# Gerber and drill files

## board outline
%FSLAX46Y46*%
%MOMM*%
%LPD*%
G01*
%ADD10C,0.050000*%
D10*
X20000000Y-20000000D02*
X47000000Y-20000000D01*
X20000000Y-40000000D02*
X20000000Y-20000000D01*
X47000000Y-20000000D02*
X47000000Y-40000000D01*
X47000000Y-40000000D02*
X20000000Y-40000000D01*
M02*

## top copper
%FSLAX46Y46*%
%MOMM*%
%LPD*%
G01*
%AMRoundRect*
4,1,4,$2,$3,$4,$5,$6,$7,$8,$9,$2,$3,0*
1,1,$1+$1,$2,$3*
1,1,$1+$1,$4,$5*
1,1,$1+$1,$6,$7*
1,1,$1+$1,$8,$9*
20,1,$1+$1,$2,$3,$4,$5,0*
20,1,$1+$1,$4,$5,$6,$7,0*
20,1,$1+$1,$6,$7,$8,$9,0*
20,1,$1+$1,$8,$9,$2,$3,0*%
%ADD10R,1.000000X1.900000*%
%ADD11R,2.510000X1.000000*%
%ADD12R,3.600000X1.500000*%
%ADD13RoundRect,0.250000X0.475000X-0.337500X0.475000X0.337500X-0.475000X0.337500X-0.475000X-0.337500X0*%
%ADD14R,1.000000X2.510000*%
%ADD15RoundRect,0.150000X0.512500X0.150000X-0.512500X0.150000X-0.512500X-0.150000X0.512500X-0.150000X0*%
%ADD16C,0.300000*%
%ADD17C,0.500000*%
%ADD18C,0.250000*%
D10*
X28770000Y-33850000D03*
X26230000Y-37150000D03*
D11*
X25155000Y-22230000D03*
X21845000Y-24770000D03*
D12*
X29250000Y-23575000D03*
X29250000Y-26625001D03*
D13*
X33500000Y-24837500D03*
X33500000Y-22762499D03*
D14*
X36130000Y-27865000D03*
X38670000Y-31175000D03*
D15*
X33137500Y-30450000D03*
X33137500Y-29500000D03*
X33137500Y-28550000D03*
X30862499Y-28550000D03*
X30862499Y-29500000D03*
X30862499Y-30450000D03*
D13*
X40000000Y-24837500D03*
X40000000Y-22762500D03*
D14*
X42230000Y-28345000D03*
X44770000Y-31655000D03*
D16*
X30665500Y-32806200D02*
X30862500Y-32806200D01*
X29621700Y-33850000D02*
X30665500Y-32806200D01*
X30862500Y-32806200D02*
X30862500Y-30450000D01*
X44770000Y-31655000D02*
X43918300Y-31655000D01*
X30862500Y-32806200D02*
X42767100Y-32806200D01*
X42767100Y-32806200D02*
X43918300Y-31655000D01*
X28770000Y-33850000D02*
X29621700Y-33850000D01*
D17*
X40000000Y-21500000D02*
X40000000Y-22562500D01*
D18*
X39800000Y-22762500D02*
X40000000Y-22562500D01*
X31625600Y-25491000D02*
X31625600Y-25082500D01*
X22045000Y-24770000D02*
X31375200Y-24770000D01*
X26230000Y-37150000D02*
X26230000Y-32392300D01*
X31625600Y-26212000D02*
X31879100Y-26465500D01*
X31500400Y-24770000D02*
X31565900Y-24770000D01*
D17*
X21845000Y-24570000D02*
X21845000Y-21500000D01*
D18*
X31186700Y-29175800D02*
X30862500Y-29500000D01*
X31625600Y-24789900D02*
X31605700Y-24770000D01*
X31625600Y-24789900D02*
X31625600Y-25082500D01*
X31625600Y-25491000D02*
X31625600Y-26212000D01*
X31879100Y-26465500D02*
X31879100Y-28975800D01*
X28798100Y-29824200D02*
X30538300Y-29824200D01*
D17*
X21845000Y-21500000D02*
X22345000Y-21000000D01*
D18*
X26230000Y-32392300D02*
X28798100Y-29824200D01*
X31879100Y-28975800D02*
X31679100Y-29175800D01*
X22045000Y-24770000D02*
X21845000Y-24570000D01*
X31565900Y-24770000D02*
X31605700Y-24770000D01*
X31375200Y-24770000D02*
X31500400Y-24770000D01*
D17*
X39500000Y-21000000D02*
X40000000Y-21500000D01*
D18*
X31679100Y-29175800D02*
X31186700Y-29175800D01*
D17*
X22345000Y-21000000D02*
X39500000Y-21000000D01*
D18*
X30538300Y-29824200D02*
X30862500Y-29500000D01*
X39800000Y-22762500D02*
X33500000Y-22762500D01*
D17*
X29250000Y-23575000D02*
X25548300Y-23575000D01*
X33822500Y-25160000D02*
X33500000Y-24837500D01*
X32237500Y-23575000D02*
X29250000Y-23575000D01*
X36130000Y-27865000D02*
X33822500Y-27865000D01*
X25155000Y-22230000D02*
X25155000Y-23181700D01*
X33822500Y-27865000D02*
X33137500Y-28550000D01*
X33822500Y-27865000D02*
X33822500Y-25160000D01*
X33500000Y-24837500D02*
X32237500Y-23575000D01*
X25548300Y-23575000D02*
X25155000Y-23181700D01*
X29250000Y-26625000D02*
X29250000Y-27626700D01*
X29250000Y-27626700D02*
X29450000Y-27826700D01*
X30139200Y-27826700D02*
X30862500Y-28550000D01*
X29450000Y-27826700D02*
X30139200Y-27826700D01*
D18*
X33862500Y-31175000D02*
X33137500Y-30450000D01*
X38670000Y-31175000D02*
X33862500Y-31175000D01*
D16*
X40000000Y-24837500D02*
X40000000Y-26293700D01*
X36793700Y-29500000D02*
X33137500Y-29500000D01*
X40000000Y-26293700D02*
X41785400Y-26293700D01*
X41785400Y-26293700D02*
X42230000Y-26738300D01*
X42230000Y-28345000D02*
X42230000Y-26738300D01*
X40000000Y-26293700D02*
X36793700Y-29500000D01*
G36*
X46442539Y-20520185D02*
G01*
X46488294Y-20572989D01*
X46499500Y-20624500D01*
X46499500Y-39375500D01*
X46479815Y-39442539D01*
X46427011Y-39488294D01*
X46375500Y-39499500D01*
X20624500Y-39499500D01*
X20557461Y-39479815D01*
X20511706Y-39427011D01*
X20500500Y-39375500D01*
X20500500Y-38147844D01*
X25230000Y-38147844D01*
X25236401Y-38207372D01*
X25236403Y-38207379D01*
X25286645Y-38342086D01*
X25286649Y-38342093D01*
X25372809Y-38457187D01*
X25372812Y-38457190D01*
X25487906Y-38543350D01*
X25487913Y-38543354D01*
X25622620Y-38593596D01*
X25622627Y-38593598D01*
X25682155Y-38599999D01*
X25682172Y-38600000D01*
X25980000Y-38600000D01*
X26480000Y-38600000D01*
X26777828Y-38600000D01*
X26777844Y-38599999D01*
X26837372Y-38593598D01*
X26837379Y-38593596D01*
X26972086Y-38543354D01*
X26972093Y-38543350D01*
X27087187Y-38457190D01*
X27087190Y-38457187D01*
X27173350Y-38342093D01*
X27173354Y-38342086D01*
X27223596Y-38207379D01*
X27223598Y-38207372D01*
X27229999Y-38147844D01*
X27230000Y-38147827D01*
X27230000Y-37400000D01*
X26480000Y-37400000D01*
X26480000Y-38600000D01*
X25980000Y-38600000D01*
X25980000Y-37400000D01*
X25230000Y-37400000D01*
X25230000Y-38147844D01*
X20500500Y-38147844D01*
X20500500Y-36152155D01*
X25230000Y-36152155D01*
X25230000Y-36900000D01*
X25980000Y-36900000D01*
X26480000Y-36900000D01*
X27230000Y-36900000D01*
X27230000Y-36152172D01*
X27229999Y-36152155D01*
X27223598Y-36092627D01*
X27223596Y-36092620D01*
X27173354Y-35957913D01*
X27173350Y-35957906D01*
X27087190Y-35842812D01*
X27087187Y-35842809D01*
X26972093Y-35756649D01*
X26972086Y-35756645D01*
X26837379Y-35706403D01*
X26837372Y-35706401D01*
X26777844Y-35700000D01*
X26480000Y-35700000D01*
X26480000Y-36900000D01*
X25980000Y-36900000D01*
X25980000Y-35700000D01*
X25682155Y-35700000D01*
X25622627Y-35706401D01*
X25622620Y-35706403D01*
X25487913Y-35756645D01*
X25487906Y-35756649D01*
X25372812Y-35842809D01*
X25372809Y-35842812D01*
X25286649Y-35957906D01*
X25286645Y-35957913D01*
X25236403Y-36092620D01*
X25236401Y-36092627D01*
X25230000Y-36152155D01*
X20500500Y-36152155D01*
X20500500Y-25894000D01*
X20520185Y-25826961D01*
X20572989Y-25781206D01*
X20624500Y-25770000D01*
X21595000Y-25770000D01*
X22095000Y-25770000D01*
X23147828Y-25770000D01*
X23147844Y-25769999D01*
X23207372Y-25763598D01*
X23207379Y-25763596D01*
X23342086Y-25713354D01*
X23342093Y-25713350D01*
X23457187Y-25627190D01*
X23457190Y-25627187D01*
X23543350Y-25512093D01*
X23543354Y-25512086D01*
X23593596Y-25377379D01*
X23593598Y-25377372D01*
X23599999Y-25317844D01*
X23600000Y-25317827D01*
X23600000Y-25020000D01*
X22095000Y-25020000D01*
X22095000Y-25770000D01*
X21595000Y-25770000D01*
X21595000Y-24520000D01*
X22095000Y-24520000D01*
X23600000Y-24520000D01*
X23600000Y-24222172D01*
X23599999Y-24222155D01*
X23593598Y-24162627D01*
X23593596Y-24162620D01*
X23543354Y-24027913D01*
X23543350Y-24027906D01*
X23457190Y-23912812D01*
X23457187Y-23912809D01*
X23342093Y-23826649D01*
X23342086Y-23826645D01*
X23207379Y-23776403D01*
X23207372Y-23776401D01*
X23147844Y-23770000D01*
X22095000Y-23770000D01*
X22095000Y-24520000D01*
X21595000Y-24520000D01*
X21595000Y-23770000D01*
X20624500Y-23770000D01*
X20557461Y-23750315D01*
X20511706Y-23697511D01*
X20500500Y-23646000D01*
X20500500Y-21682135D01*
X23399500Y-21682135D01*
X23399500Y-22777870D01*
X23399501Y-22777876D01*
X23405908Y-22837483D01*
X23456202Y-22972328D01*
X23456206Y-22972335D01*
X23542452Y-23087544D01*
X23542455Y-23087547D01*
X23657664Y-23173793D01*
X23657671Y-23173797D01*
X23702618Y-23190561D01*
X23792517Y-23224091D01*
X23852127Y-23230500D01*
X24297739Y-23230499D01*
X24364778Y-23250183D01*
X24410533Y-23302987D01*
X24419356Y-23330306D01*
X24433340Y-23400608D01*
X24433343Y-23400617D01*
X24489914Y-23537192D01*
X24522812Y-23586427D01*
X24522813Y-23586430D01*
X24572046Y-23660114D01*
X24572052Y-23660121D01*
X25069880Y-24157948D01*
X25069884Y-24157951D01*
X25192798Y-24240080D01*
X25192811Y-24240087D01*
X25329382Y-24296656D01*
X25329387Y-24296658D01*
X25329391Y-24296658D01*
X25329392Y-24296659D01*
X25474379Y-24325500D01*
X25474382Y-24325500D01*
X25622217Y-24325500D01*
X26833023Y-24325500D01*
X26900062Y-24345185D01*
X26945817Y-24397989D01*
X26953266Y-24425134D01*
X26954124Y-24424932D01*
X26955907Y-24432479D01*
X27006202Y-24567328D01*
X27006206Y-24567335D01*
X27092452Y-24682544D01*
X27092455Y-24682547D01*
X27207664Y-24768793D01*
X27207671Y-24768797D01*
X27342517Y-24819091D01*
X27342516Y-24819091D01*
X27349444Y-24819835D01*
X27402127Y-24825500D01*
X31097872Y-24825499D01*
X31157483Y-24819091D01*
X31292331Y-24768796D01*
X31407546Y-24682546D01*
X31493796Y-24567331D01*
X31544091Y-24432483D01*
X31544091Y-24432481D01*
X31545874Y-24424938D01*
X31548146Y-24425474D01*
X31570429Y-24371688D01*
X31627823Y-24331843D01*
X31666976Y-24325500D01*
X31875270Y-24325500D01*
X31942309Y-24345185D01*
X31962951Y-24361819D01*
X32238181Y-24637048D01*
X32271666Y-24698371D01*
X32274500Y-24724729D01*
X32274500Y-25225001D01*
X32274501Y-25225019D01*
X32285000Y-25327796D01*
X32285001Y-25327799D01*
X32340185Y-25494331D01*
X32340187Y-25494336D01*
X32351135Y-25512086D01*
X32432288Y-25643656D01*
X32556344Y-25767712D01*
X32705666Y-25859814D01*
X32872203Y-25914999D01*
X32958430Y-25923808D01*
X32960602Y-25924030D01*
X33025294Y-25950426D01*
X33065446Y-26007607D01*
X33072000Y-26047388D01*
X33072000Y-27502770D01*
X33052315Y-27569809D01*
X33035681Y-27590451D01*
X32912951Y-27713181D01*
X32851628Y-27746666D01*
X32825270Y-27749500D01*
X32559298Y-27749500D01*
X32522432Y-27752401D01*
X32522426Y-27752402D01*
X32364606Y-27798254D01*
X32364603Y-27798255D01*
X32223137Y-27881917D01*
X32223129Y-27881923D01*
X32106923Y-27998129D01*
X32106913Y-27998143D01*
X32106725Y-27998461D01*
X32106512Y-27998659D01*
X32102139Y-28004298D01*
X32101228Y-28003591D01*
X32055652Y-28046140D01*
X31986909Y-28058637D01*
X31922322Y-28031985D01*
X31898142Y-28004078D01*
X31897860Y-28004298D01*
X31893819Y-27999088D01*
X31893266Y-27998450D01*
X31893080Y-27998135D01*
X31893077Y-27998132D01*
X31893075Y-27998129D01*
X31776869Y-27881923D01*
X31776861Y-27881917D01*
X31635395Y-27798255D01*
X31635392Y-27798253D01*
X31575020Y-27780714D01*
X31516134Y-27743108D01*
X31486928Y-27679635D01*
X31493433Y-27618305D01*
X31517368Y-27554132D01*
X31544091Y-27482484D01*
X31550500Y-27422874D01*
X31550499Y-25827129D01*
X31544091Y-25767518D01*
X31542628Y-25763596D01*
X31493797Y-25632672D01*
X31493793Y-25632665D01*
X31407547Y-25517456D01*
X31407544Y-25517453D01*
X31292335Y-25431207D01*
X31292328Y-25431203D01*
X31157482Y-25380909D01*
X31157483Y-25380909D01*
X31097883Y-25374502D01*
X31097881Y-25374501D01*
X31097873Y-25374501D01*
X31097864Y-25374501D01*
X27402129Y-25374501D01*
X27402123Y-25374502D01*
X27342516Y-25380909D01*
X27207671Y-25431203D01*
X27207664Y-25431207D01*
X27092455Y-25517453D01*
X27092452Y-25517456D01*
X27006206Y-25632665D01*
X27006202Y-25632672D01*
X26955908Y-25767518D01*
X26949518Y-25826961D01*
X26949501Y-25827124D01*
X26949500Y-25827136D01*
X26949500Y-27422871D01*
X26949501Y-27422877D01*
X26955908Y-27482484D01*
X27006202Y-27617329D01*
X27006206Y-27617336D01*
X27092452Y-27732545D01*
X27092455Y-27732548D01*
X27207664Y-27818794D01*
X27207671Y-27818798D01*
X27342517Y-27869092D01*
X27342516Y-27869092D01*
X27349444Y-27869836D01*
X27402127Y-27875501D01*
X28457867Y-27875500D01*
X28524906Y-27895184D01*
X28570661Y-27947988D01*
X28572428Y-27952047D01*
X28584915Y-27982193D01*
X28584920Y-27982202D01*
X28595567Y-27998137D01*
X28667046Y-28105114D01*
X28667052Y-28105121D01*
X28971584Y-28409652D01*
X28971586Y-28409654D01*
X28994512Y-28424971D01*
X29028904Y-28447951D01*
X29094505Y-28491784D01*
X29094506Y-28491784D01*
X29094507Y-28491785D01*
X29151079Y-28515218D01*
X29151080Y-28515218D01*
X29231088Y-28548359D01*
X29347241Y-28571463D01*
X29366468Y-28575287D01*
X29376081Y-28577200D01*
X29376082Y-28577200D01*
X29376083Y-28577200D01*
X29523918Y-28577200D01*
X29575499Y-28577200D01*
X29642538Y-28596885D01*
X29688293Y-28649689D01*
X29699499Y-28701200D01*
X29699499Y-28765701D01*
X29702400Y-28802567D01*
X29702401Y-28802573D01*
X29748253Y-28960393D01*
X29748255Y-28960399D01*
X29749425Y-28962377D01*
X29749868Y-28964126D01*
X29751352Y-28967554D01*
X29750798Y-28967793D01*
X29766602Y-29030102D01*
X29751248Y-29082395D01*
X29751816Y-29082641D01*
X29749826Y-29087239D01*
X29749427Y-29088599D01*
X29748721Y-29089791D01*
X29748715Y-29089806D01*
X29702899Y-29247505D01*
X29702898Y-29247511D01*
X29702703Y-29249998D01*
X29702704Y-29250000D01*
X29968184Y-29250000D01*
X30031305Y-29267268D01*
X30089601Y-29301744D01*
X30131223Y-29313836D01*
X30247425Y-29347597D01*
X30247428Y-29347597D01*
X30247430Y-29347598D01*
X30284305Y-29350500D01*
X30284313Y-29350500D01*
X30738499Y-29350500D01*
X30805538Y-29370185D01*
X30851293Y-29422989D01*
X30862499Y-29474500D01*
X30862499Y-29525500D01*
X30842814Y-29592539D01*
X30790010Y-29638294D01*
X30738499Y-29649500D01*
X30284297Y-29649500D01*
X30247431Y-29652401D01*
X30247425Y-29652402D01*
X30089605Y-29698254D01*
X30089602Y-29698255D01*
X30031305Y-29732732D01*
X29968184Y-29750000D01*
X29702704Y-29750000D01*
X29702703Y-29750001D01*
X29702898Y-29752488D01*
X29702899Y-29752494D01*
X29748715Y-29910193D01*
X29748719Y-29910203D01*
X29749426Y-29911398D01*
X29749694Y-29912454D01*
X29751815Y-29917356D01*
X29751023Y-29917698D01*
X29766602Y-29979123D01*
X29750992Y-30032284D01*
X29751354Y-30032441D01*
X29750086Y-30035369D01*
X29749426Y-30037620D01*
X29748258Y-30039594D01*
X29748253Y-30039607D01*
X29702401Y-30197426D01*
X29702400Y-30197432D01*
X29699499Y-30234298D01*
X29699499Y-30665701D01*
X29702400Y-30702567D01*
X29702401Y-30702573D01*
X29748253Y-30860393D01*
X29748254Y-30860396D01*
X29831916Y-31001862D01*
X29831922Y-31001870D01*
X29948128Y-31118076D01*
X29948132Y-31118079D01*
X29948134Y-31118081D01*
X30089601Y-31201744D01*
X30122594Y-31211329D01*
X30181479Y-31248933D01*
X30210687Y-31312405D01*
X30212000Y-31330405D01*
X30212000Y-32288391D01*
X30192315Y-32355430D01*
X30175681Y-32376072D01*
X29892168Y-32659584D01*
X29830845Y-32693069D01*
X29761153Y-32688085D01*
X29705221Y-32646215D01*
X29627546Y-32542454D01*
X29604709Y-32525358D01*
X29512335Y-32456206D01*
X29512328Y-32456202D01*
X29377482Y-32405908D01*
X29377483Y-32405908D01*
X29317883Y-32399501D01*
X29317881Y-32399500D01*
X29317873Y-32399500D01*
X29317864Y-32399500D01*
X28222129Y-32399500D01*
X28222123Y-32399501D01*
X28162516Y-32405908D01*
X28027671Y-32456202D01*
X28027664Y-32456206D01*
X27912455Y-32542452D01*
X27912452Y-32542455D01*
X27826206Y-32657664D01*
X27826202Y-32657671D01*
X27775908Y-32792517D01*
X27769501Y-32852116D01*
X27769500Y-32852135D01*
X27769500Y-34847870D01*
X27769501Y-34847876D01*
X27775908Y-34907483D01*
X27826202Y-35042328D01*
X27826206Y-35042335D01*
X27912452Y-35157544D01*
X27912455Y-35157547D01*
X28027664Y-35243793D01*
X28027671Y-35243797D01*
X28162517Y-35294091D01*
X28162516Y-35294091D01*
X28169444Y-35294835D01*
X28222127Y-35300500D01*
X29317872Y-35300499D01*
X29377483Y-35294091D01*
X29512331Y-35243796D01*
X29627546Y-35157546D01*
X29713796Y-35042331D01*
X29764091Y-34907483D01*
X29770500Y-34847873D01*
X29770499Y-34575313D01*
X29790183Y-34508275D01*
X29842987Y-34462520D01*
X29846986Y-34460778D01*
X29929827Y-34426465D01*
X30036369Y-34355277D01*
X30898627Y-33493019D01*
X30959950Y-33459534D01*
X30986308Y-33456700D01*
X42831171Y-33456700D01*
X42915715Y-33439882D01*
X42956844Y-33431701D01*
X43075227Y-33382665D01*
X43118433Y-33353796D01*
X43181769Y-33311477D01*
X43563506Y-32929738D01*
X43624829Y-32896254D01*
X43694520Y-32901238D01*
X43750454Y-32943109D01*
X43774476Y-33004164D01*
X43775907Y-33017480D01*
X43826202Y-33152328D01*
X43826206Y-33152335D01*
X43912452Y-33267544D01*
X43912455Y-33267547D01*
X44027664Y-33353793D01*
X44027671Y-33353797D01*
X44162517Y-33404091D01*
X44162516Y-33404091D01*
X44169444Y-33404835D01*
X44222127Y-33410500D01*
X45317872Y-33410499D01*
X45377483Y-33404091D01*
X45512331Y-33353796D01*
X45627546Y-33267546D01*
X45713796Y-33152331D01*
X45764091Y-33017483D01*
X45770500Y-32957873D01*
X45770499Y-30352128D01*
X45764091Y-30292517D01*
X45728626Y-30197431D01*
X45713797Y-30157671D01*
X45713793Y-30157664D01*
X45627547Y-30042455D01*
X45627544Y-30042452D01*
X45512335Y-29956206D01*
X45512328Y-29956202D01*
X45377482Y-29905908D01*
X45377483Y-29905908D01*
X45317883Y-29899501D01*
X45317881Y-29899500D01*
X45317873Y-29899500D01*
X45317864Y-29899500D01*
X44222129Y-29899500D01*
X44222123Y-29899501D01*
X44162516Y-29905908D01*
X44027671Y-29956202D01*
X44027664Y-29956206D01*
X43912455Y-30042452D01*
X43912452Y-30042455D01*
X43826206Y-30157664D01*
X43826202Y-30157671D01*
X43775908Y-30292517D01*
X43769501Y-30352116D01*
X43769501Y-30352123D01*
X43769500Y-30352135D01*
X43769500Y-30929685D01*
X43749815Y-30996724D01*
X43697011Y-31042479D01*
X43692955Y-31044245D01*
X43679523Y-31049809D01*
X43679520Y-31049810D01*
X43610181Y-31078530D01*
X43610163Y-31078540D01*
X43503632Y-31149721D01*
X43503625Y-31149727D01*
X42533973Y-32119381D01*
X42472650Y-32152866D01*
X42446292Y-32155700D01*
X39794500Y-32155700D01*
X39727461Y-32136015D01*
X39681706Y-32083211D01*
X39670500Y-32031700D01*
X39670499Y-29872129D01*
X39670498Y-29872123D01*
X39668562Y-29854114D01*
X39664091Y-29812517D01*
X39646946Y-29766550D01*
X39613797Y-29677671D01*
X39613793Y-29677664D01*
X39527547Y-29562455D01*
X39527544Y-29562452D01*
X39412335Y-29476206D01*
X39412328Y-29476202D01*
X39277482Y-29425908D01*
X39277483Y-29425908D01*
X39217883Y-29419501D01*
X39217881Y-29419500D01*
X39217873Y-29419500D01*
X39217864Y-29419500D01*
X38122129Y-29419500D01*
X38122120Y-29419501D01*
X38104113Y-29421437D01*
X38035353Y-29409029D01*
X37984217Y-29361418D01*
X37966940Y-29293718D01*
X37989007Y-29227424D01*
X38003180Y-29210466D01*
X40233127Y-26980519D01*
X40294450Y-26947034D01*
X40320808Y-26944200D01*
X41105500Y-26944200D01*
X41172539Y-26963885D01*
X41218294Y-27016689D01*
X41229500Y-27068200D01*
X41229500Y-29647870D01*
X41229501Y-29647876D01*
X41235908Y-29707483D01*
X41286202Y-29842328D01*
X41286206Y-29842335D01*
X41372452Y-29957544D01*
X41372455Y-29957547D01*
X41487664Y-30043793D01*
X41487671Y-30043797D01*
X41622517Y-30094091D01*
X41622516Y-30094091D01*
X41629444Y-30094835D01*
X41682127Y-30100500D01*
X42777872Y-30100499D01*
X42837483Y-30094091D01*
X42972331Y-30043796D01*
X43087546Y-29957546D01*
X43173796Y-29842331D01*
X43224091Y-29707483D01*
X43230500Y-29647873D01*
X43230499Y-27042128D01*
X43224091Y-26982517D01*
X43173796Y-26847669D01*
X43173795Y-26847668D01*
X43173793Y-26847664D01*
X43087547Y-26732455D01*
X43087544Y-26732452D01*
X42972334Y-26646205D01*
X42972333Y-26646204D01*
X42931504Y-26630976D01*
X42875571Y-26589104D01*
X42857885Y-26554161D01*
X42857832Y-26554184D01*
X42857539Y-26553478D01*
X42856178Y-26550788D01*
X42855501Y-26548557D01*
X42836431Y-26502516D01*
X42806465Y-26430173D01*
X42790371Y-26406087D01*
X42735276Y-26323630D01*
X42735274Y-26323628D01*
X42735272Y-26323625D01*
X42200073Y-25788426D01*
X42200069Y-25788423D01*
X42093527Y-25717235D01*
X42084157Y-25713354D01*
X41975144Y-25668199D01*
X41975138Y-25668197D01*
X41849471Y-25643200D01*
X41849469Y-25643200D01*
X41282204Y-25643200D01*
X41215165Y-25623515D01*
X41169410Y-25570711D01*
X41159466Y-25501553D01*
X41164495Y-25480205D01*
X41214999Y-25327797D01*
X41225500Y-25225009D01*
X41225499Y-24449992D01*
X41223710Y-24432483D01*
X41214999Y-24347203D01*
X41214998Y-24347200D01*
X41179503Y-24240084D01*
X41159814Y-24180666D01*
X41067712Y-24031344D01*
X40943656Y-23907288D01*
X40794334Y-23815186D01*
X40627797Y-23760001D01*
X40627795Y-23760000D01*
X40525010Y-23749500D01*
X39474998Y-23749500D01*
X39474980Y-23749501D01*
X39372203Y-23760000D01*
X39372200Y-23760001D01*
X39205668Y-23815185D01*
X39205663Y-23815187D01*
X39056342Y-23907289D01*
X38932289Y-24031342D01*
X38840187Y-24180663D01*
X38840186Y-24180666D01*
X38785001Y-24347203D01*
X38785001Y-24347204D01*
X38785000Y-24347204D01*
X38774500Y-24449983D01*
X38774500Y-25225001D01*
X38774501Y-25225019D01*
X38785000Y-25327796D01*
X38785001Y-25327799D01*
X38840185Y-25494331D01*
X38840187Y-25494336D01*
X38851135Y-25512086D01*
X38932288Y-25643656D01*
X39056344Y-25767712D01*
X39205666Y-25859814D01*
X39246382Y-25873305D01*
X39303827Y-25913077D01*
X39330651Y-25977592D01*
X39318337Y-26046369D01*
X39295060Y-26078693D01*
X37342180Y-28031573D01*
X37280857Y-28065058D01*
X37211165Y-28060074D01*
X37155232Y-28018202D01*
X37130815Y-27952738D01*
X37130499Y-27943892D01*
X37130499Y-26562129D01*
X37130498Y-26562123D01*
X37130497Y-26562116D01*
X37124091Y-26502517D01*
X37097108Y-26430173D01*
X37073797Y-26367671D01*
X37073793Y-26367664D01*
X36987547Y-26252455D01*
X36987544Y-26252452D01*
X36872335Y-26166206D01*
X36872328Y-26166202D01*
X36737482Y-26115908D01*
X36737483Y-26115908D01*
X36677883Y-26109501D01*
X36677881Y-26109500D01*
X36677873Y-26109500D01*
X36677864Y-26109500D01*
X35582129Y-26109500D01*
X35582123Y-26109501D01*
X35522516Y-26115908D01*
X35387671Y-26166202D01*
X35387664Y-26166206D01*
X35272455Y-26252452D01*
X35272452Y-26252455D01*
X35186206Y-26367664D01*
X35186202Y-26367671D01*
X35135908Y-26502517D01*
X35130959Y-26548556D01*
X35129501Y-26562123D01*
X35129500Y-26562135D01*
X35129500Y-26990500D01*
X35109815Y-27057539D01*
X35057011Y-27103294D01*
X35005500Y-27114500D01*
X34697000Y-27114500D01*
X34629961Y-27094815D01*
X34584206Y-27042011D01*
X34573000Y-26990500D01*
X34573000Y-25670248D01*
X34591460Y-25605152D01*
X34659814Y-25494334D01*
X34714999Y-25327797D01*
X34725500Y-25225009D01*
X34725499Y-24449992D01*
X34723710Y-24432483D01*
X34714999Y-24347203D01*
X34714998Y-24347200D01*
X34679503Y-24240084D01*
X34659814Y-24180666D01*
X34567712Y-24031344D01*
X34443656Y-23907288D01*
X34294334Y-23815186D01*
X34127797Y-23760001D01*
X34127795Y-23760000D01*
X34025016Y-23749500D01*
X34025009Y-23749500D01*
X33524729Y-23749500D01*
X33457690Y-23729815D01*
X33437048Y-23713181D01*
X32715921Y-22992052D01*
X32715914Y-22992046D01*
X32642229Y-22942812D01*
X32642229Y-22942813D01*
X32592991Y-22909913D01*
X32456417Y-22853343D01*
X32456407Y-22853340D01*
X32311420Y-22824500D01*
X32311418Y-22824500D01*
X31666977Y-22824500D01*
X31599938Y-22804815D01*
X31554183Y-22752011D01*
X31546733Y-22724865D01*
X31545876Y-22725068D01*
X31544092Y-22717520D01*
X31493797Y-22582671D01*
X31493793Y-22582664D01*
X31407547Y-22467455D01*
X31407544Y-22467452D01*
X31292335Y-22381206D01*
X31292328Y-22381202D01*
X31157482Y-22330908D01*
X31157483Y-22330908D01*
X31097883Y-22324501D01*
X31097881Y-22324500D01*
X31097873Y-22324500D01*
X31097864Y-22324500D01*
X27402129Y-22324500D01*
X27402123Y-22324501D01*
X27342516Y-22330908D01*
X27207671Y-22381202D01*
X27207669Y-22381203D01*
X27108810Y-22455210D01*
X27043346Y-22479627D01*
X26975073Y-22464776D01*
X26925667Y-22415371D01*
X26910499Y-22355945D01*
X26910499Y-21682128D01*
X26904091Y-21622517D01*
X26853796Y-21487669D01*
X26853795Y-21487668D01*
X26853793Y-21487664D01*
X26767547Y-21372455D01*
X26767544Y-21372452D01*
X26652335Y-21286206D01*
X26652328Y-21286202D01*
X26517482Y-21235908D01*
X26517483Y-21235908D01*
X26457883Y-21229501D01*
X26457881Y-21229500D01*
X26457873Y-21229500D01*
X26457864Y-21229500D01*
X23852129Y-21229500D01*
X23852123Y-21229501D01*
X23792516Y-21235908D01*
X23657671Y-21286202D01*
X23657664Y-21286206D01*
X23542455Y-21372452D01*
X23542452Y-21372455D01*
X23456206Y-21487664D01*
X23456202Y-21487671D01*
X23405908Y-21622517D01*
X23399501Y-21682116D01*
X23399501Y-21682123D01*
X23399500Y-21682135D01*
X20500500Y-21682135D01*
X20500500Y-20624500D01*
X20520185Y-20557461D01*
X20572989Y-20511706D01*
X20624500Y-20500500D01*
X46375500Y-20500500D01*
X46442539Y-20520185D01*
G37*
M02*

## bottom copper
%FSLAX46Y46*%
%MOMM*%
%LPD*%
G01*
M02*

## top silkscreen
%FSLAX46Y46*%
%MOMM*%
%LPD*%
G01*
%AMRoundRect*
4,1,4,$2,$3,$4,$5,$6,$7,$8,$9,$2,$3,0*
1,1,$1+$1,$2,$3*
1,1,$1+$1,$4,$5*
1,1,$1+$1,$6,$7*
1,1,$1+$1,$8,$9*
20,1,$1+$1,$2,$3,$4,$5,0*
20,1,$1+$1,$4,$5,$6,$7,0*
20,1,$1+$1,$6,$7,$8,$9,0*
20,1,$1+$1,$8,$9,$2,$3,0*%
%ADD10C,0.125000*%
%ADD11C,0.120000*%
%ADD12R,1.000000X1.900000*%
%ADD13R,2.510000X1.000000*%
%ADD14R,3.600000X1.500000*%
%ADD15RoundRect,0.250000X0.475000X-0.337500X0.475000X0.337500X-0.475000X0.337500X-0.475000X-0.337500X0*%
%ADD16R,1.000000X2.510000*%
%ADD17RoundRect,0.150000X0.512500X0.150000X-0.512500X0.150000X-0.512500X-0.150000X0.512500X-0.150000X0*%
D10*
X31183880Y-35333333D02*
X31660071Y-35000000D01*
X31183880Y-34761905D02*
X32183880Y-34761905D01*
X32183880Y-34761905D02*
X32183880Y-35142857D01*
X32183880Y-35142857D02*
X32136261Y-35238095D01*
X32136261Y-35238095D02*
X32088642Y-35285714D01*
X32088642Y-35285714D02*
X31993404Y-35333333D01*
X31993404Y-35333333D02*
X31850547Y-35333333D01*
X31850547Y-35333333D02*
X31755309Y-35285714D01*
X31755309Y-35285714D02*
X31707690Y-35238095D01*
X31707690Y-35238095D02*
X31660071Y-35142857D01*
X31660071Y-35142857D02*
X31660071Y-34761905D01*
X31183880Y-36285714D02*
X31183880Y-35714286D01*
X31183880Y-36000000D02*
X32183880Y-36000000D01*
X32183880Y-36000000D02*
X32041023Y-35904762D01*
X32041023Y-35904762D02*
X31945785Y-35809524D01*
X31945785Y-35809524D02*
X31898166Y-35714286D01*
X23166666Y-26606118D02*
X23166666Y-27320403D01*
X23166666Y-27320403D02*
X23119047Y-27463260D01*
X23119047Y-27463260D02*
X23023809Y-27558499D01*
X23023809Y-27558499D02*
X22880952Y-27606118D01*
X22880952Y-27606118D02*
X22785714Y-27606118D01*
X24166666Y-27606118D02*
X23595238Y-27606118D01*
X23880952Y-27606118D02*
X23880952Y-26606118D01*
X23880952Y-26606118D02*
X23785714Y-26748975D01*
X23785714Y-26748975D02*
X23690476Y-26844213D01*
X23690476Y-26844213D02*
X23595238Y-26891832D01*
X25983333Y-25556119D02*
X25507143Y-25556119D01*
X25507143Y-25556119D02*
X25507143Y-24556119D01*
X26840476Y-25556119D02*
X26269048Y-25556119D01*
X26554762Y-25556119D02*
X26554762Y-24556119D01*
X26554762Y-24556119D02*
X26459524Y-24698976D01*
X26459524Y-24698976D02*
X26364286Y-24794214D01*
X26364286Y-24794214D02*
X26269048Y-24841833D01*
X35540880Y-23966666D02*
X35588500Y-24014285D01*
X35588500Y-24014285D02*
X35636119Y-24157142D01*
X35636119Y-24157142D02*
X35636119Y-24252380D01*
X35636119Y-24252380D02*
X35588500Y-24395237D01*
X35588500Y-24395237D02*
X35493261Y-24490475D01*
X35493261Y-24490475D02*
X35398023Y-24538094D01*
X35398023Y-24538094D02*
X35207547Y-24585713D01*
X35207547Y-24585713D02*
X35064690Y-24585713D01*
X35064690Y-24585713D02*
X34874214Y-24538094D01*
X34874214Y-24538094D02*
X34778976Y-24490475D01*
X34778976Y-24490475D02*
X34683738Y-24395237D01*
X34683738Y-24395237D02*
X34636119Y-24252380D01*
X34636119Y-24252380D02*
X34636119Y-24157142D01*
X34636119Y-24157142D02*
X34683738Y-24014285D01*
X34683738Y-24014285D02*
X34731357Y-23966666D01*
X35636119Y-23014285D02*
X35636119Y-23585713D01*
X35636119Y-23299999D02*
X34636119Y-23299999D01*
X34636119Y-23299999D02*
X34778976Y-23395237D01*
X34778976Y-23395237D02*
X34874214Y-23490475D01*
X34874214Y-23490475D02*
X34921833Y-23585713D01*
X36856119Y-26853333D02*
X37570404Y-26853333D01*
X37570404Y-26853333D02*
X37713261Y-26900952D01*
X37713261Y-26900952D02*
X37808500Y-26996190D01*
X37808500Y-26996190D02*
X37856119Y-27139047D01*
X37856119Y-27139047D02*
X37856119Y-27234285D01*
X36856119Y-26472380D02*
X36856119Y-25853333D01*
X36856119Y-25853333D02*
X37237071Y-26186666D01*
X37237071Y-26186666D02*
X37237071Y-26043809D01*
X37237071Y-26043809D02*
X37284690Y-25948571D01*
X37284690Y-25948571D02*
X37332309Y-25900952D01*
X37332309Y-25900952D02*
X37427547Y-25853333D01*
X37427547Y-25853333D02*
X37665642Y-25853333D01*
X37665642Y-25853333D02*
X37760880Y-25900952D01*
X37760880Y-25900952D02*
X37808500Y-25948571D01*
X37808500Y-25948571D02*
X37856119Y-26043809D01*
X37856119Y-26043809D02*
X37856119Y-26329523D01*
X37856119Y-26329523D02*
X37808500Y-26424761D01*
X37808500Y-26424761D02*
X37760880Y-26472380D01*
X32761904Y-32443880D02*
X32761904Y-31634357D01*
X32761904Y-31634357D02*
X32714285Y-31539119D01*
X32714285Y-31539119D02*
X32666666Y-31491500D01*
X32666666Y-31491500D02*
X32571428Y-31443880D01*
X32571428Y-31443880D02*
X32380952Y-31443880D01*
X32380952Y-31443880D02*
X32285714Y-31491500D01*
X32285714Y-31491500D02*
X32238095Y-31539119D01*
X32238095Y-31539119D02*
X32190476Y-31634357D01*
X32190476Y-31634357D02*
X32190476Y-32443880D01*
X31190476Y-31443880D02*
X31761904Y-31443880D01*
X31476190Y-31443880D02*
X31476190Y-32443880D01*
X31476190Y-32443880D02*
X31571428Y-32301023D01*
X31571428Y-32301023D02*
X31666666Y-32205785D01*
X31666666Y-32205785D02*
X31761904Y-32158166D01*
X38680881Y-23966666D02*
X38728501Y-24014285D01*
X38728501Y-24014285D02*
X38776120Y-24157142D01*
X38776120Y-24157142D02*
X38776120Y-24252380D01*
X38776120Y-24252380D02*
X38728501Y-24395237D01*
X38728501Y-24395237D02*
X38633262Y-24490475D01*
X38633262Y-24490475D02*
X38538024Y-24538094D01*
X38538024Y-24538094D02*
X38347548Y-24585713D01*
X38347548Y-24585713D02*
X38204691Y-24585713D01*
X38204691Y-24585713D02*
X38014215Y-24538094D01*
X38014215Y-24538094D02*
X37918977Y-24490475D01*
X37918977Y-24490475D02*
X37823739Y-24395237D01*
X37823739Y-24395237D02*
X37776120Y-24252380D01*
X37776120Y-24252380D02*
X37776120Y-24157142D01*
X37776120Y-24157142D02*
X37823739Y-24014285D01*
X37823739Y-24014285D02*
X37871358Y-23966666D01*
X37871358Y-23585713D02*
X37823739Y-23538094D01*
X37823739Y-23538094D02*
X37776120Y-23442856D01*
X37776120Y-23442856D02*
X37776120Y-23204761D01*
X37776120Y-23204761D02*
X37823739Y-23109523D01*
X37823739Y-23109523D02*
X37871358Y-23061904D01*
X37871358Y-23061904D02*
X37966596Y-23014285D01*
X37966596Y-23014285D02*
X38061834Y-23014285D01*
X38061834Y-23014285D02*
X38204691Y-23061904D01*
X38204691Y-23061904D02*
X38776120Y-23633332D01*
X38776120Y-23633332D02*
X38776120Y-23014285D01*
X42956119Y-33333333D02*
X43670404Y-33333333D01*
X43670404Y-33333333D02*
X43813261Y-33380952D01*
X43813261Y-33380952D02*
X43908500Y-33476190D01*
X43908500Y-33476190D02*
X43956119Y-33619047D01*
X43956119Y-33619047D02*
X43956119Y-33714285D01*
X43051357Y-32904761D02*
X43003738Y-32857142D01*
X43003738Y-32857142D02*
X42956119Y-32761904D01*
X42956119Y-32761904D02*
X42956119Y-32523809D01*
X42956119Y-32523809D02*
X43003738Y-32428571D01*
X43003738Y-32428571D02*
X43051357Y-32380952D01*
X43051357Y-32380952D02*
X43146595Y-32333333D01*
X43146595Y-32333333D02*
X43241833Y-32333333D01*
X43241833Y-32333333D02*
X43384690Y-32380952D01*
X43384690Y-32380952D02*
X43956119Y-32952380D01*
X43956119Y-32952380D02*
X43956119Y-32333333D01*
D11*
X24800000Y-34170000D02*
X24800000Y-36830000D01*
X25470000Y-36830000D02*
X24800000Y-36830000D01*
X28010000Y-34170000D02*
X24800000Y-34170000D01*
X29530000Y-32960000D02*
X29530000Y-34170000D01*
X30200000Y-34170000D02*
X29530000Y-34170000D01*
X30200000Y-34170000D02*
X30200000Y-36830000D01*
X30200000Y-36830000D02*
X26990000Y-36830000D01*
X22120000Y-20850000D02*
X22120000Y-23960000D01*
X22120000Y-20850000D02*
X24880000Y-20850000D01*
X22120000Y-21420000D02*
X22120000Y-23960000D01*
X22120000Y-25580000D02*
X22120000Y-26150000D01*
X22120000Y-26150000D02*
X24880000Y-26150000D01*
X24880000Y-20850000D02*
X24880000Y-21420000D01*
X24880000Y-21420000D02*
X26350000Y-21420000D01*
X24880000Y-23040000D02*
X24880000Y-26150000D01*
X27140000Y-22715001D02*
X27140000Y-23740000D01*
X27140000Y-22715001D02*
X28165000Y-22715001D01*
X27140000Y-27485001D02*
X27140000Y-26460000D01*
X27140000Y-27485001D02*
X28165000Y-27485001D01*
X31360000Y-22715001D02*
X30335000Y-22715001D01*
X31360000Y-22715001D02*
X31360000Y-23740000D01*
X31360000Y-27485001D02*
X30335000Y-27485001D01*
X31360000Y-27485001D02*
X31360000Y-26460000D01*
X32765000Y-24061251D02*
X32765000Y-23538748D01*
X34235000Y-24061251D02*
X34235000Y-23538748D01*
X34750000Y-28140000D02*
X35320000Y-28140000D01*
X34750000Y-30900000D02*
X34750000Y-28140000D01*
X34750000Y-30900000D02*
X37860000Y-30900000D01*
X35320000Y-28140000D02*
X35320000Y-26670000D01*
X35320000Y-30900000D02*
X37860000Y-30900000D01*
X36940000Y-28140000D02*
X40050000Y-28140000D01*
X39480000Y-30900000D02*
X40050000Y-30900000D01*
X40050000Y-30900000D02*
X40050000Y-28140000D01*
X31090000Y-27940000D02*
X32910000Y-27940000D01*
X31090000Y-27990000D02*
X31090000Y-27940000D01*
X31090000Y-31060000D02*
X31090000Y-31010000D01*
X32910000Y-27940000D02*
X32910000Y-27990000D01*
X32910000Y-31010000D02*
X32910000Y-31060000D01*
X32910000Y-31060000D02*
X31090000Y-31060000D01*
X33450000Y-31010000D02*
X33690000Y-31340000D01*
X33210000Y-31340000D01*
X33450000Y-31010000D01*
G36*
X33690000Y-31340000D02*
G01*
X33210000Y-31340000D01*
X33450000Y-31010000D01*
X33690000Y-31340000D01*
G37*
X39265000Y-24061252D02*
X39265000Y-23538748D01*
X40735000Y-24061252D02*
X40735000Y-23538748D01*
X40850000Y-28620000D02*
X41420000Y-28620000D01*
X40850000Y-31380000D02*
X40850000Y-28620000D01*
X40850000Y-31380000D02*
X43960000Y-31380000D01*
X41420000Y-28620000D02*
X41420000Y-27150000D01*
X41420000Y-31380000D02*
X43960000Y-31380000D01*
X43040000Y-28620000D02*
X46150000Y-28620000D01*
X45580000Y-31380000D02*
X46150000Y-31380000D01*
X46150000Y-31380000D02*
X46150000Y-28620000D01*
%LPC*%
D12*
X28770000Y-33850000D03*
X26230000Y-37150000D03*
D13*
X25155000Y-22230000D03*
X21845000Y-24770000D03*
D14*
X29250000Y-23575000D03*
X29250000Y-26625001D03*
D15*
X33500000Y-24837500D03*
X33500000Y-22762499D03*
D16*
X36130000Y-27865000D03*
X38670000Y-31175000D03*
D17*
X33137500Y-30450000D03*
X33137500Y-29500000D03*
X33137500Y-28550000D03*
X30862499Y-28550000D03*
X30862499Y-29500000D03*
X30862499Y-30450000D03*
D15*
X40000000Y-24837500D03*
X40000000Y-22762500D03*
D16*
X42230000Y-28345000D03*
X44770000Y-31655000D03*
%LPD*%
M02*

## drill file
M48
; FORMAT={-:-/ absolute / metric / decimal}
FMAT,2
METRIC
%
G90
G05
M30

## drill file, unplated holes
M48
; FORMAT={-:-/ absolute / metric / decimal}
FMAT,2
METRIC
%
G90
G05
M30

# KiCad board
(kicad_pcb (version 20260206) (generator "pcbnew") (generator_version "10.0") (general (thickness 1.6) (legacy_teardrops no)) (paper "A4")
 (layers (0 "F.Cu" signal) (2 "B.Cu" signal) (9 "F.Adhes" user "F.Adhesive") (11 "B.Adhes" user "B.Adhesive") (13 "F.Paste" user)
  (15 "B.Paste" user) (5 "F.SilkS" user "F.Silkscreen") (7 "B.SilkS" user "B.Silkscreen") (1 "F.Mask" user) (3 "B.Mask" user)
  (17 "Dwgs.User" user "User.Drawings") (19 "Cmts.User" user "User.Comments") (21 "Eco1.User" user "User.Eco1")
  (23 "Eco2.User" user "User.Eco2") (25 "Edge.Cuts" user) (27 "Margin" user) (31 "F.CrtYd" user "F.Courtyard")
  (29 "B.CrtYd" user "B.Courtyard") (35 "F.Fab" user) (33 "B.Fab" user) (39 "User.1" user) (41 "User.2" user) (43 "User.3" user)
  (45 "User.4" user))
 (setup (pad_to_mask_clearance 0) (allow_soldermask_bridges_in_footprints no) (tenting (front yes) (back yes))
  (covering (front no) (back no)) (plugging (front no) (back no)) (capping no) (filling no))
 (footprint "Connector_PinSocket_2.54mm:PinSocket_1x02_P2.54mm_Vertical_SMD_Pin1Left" (layer "F.Cu") (at 27.5 35.5 -90)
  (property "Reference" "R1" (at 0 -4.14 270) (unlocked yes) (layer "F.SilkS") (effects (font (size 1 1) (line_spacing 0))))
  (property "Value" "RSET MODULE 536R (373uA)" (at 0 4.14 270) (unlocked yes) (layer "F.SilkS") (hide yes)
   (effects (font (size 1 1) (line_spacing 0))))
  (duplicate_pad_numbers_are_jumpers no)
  (fp_line (start -1.33 2.7) (end 1.33 2.7) (stroke (width 0.12) (type solid)) (layer "F.SilkS"))
  (fp_line (start 1.33 2.03) (end 1.33 2.7) (stroke (width 0.12) (type solid)) (layer "F.SilkS"))
  (fp_line (start -1.33 -0.51) (end -1.33 2.7) (stroke (width 0.12) (type solid)) (layer "F.SilkS"))
  (fp_line (start -2.54 -2.03) (end -1.33 -2.03) (stroke (width 0.12) (type solid)) (layer "F.SilkS"))
  (fp_line (start -1.33 -2.7) (end -1.33 -2.03) (stroke (width 0.12) (type solid)) (layer "F.SilkS"))
  (fp_line (start -1.33 -2.7) (end 1.33 -2.7) (stroke (width 0.12) (type solid)) (layer "F.SilkS"))
  (fp_line (start 1.33 -2.7) (end 1.33 0.51) (stroke (width 0.12) (type solid)) (layer "F.SilkS"))
  (pad "1" smd rect (at -1.65 -1.27 270) (size 1.9 1) (layers "F.Cu" "F.Mask" "F.Paste") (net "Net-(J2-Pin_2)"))
  (pad "2" smd rect (at 1.65 1.27 270) (size 1.9 1) (layers "F.Cu" "F.Mask" "F.Paste") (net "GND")))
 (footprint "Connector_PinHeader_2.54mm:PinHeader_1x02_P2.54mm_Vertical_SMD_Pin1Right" (layer "F.Cu") (at 23.5 23.5)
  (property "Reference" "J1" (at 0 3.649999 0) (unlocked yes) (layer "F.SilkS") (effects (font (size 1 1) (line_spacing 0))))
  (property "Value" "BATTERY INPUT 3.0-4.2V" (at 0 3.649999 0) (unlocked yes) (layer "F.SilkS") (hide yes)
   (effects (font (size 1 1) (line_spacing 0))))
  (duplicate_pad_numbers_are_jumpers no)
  (fp_line (start -1.38 -2.65) (end -1.38 0.46) (stroke (width 0.12) (type solid)) (layer "F.SilkS"))
  (fp_line (start -1.38 -2.65) (end 1.38 -2.65) (stroke (width 0.12) (type solid)) (layer "F.SilkS"))
  (fp_line (start -1.38 -2.08) (end -1.38 0.46) (stroke (width 0.12) (type solid)) (layer "F.SilkS"))
  (fp_line (start -1.38 2.08) (end -1.38 2.65) (stroke (width 0.12) (type solid)) (layer "F.SilkS"))
  (fp_line (start -1.38 2.65) (end 1.38 2.65) (stroke (width 0.12) (type solid)) (layer "F.SilkS"))
  (fp_line (start 1.38 -2.65) (end 1.38 -2.08) (stroke (width 0.12) (type solid)) (layer "F.SilkS"))
  (fp_line (start 1.38 -2.08) (end 2.85 -2.08) (stroke (width 0.12) (type solid)) (layer "F.SilkS"))
  (fp_line (start 1.38 -0.46) (end 1.38 2.65) (stroke (width 0.12) (type solid)) (layer "F.SilkS"))
  (pad "1" smd rect (at 1.655 -1.27) (size 2.51 1) (layers "F.Cu" "F.Mask" "F.Paste") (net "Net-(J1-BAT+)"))
  (pad "2" smd rect (at -1.655 1.27) (size 2.51 1) (layers "F.Cu" "F.Mask" "F.Paste") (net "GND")))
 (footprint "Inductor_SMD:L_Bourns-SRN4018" (layer "F.Cu") (at 29.25 25.1 -90)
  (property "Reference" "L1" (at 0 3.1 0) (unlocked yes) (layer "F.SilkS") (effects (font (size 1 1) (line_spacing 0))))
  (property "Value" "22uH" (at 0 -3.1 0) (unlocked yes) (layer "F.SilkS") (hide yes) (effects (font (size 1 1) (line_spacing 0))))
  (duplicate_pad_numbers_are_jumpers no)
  (fp_line (start -2.384999 2.11) (end -1.36 2.11) (stroke (width 0.12) (type solid)) (layer "F.SilkS"))
  (fp_line (start -2.384999 2.11) (end -2.384999 1.085) (stroke (width 0.12) (type solid)) (layer "F.SilkS"))
  (fp_line (start 2.385001 2.11) (end 1.36 2.11) (stroke (width 0.12) (type solid)) (layer "F.SilkS"))
  (fp_line (start 2.385001 2.11) (end 2.385001 1.085) (stroke (width 0.12) (type solid)) (layer "F.SilkS"))
  (fp_line (start -2.384999 -2.11) (end -2.384999 -1.085) (stroke (width 0.12) (type solid)) (layer "F.SilkS"))
  (fp_line (start -2.384999 -2.11) (end -1.36 -2.11) (stroke (width 0.12) (type solid)) (layer "F.SilkS"))
  (fp_line (start 2.385001 -2.11) (end 2.385001 -1.085) (stroke (width 0.12) (type solid)) (layer "F.SilkS"))
  (fp_line (start 2.385001 -2.11) (end 1.36 -2.11) (stroke (width 0.12) (type solid)) (layer "F.SilkS"))
  (pad "1" smd rect (at -1.525 0 270) (size 1.5 3.6) (layers "F.Cu" "F.Mask" "F.Paste") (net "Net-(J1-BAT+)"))
  (pad "2" smd rect (at 1.525001 0 270) (size 1.5 3.6) (layers "F.Cu" "F.Mask" "F.Paste") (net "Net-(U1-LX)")))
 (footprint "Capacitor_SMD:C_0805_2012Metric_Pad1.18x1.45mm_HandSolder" (layer "F.Cu") (at 33.5 23.8 90)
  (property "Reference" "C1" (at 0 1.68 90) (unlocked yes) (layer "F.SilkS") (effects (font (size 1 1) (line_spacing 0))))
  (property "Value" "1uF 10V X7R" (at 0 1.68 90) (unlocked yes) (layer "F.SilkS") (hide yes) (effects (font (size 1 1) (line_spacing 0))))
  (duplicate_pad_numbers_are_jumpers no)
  (fp_line (start -0.261251 -0.735) (end 0.261252 -0.735) (stroke (width 0.12) (type solid)) (layer "F.SilkS"))
  (fp_line (start -0.261251 0.735) (end 0.261252 0.735) (stroke (width 0.12) (type solid)) (layer "F.SilkS"))
  (pad "1" smd roundrect (at -1.0375 0 90) (size 1.175 1.45) (layers "F.Cu" "F.Mask" "F.Paste") (roundrect_rratio 0.212766)
   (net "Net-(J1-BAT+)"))
  (pad "2" smd roundrect (at 1.037501 0 90) (size 1.175 1.45) (layers "F.Cu" "F.Mask" "F.Paste") (roundrect_rratio 0.212766) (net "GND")
   (zone_connect 3)))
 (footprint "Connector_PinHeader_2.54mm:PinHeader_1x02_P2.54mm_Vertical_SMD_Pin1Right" (layer "F.Cu") (at 37.4 29.52 90)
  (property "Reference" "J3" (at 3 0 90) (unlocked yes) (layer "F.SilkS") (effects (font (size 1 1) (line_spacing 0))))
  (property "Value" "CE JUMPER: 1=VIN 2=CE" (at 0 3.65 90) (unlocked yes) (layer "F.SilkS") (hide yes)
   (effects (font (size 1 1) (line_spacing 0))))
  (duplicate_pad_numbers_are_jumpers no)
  (fp_line (start 1.38 -2.65) (end 1.38 -2.08) (stroke (width 0.12) (type solid)) (layer "F.SilkS"))
  (fp_line (start -1.38 -2.65) (end 1.38 -2.65) (stroke (width 0.12) (type solid)) (layer "F.SilkS"))
  (fp_line (start -1.38 -2.65) (end -1.38 0.46) (stroke (width 0.12) (type solid)) (layer "F.SilkS"))
  (fp_line (start 1.38 -2.08) (end 2.85 -2.08) (stroke (width 0.12) (type solid)) (layer "F.SilkS"))
  (fp_line (start -1.38 -2.08) (end -1.38 0.46) (stroke (width 0.12) (type solid)) (layer "F.SilkS"))
  (fp_line (start 1.38 -0.46) (end 1.38 2.65) (stroke (width 0.12) (type solid)) (layer "F.SilkS"))
  (fp_line (start -1.38 2.08) (end -1.38 2.65) (stroke (width 0.12) (type solid)) (layer "F.SilkS"))
  (fp_line (start -1.38 2.65) (end 1.38 2.65) (stroke (width 0.12) (type solid)) (layer "F.SilkS"))
  (pad "1" smd rect (at 1.655 -1.27 90) (size 2.51 1) (layers "F.Cu" "F.Mask" "F.Paste") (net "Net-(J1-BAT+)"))
  (pad "2" smd rect (at -1.655 1.27 90) (size 2.51 1) (layers "F.Cu" "F.Mask" "F.Paste") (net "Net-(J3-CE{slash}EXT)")))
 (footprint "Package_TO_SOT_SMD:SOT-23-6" (layer "F.Cu") (at 32 29.5 180)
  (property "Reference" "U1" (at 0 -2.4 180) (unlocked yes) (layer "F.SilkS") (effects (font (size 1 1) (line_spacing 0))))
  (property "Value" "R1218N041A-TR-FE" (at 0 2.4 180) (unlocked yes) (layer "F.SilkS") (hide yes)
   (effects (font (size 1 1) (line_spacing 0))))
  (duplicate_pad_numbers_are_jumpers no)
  (fp_line (start 0.91 1.56) (end -0.91 1.56) (stroke (width 0.12) (type solid)) (layer "F.SilkS"))
  (fp_line (start 0.91 1.51) (end 0.91 1.56) (stroke (width 0.12) (type solid)) (layer "F.SilkS"))
  (fp_line (start 0.91 -1.56) (end 0.91 -1.51) (stroke (width 0.12) (type solid)) (layer "F.SilkS"))
  (fp_line (start -0.91 1.56) (end -0.91 1.51) (stroke (width 0.12) (type solid)) (layer "F.SilkS"))
  (fp_line (start -0.91 -1.51) (end -0.91 -1.56) (stroke (width 0.12) (type solid)) (layer "F.SilkS"))
  (fp_line (start -0.91 -1.56) (end 0.91 -1.56) (stroke (width 0.12) (type solid)) (layer "F.SilkS"))
  (fp_poly (pts (xy -1.45 -1.51) (xy -1.69 -1.84) (xy -1.21 -1.84)) (stroke (width 0.12) (type solid)) (fill yes) (layer "F.SilkS"))
  (pad "1" smd roundrect (at -1.1375 -0.95 180) (size 1.325 0.6) (layers "F.Cu" "F.Mask" "F.Paste") (roundrect_rratio 0.25)
   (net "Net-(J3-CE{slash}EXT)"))
  (pad "2" smd roundrect (at -1.1375 0 180) (size 1.325 0.6) (layers "F.Cu" "F.Mask" "F.Paste") (roundrect_rratio 0.25)
   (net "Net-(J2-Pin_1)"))
  (pad "3" smd roundrect (at -1.1375 0.95 180) (size 1.325 0.6) (layers "F.Cu" "F.Mask" "F.Paste") (roundrect_rratio 0.25)
   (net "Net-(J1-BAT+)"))
  (pad "4" smd roundrect (at 1.137501 0.95 180) (size 1.325 0.6) (layers "F.Cu" "F.Mask" "F.Paste") (roundrect_rratio 0.25)
   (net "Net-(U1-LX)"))
  (pad "5" smd roundrect (at 1.137501 0 180) (size 1.325 0.6) (layers "F.Cu" "F.Mask" "F.Paste") (roundrect_rratio 0.25) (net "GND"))
  (pad "6" smd roundrect (at 1.137501 -0.95 180) (size 1.325 0.6) (layers "F.Cu" "F.Mask" "F.Paste") (roundrect_rratio 0.25)
   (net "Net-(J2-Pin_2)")))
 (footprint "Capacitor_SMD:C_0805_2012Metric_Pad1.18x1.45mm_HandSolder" (layer "F.Cu") (at 40 23.8 90)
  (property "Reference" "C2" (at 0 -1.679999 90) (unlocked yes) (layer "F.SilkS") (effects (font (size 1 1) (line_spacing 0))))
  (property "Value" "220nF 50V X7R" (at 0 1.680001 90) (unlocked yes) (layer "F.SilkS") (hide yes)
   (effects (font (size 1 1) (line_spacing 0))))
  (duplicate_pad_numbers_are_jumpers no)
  (fp_line (start -0.261252 -0.735) (end 0.261252 -0.735) (stroke (width 0.12) (type solid)) (layer "F.SilkS"))
  (fp_line (start -0.261252 0.735) (end 0.261252 0.735) (stroke (width 0.12) (type solid)) (layer "F.SilkS"))
  (pad "1" smd roundrect (at -1.0375 0 90) (size 1.175 1.45) (layers "F.Cu" "F.Mask" "F.Paste") (roundrect_rratio 0.212766)
   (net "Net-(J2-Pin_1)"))
  (pad "2" smd roundrect (at 1.0375 0 90) (size 1.175 1.45) (layers "F.Cu" "F.Mask" "F.Paste") (roundrect_rratio 0.212766) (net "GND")
   (zone_connect 3)))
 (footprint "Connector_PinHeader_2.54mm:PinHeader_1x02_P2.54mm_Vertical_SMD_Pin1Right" (layer "F.Cu") (at 43.5 30 90)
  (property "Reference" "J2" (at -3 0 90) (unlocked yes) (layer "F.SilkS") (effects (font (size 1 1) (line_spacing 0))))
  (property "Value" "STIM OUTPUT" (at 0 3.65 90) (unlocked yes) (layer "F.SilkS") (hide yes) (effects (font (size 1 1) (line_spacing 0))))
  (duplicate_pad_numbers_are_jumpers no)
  (fp_line (start 1.38 -2.65) (end 1.38 -2.08) (stroke (width 0.12) (type solid)) (layer "F.SilkS"))
  (fp_line (start -1.38 -2.65) (end 1.38 -2.65) (stroke (width 0.12) (type solid)) (layer "F.SilkS"))
  (fp_line (start -1.38 -2.65) (end -1.38 0.46) (stroke (width 0.12) (type solid)) (layer "F.SilkS"))
  (fp_line (start 1.38 -2.08) (end 2.85 -2.08) (stroke (width 0.12) (type solid)) (layer "F.SilkS"))
  (fp_line (start -1.38 -2.08) (end -1.38 0.46) (stroke (width 0.12) (type solid)) (layer "F.SilkS"))
  (fp_line (start 1.38 -0.46) (end 1.38 2.65) (stroke (width 0.12) (type solid)) (layer "F.SilkS"))
  (fp_line (start -1.38 2.08) (end -1.38 2.65) (stroke (width 0.12) (type solid)) (layer "F.SilkS"))
  (fp_line (start -1.38 2.65) (end 1.38 2.65) (stroke (width 0.12) (type solid)) (layer "F.SilkS"))
  (pad "1" smd rect (at 1.655 -1.27 90) (size 2.51 1) (layers "F.Cu" "F.Mask" "F.Paste") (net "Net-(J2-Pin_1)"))
  (pad "2" smd rect (at -1.655 1.27 90) (size 2.51 1) (layers "F.Cu" "F.Mask" "F.Paste") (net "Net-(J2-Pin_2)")))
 (gr_line (start 20 20) (end 47 20) (stroke (width 0.05) (type default)) (layer "Edge.Cuts"))
 (gr_line (start 20 40) (end 20 20) (stroke (width 0.05) (type default)) (layer "Edge.Cuts"))
 (gr_line (start 47 20) (end 47 40) (stroke (width 0.05) (type default)) (layer "Edge.Cuts"))
 (gr_line (start 47 40) (end 20 40) (stroke (width 0.05) (type default)) (layer "Edge.Cuts"))
 (segment (start 30.6655 32.8062) (end 30.8625 32.8062) (width 0.3) (layer "F.Cu") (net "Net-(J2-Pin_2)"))
 (segment (start 29.6217 33.85) (end 30.6655 32.8062) (width 0.3) (layer "F.Cu") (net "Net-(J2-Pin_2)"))
 (segment (start 30.8625 32.8062) (end 30.8625 30.45) (width 0.3) (layer "F.Cu") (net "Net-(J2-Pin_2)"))
 (segment (start 44.77 31.655) (end 43.9183 31.655) (width 0.3) (layer "F.Cu") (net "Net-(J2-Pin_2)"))
 (segment (start 30.8625 32.8062) (end 42.7671 32.8062) (width 0.3) (layer "F.Cu") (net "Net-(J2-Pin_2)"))
 (segment (start 42.7671 32.8062) (end 43.9183 31.655) (width 0.3) (layer "F.Cu") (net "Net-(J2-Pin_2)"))
 (segment (start 28.77 33.85) (end 29.6217 33.85) (width 0.3) (layer "F.Cu") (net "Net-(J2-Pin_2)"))
 (segment (start 31.6256 25.491) (end 31.6256 25.0825) (width 0.25) (layer "F.Cu") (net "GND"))
 (segment (start 22.045000 24.770000) (end 31.3752 24.77) (width 0.25) (layer "F.Cu") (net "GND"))
 (segment (start 26.23 37.15) (end 26.23 32.3923) (width 0.25) (layer "F.Cu") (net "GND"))
 (segment (start 31.6256 26.212) (end 31.8791 26.4655) (width 0.25) (layer "F.Cu") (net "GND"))
 (segment (start 31.5004 24.77) (end 31.5659 24.77) (width 0.25) (layer "F.Cu") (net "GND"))
 (segment (start 31.1867 29.1758) (end 30.8625 29.5) (width 0.25) (layer "F.Cu") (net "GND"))
 (segment (start 31.625600 24.789900) (end 31.6256 25.0825) (width 0.25) (layer "F.Cu") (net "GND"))
 (segment (start 31.6256 25.491) (end 31.6256 26.212) (width 0.25) (layer "F.Cu") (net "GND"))
 (segment (start 31.8791 26.4655) (end 31.879100 28.975800) (width 0.25) (layer "F.Cu") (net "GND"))
 (segment (start 28.7981 29.8242) (end 30.5383 29.8242) (width 0.25) (layer "F.Cu") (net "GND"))
 (segment (start 26.23 32.3923) (end 28.7981 29.8242) (width 0.25) (layer "F.Cu") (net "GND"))
 (segment (start 31.5659 24.77) (end 31.605700 24.770000) (width 0.25) (layer "F.Cu") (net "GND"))
 (segment (start 31.3752 24.77) (end 31.5004 24.77) (width 0.25) (layer "F.Cu") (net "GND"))
 (segment (start 31.679100 29.175800) (end 31.1867 29.1758) (width 0.25) (layer "F.Cu") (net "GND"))
 (segment (start 30.5383 29.8242) (end 30.8625 29.5) (width 0.25) (layer "F.Cu") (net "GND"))
 (segment (start 39.800000 22.762500) (end 33.5 22.7625) (width 0.25) (layer "F.Cu") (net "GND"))
 (segment (start 29.25 23.575) (end 25.5483 23.575) (width 0.5) (layer "F.Cu") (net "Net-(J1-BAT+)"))
 (segment (start 33.8225 25.16) (end 33.5 24.8375) (width 0.5) (layer "F.Cu") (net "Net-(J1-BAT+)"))
 (segment (start 32.2375 23.575) (end 29.25 23.575) (width 0.5) (layer "F.Cu") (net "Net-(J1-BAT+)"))
 (segment (start 36.13 27.865) (end 33.8225 27.865) (width 0.5) (layer "F.Cu") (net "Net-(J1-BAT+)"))
 (segment (start 25.155 22.23) (end 25.155 23.1817) (width 0.5) (layer "F.Cu") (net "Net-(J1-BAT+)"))
 (segment (start 33.8225 27.865) (end 33.1375 28.55) (width 0.5) (layer "F.Cu") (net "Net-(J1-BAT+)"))
 (segment (start 33.8225 27.865) (end 33.8225 25.16) (width 0.5) (layer "F.Cu") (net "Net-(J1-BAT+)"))
 (segment (start 33.5 24.8375) (end 32.2375 23.575) (width 0.5) (layer "F.Cu") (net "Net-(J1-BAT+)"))
 (segment (start 25.5483 23.575) (end 25.155 23.1817) (width 0.5) (layer "F.Cu") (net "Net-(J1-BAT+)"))
 (segment (start 29.25 26.625) (end 29.250000 27.626700) (width 0.5) (layer "F.Cu") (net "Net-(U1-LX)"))
 (segment (start 30.1392 27.8267) (end 30.8625 28.55) (width 0.5) (layer "F.Cu") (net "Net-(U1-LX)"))
 (segment (start 29.450000 27.826700) (end 30.1392 27.8267) (width 0.5) (layer "F.Cu") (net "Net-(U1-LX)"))
 (segment (start 33.8625 31.175) (end 33.1375 30.45) (width 0.25) (layer "F.Cu") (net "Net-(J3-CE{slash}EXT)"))
 (segment (start 38.67 31.175) (end 33.8625 31.175) (width 0.25) (layer "F.Cu") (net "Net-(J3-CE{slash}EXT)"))
 (segment (start 40 24.8375) (end 40 26.2937) (width 0.3) (layer "F.Cu") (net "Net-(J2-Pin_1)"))
 (segment (start 36.7937 29.5) (end 33.1375 29.5) (width 0.3) (layer "F.Cu") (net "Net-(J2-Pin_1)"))
 (segment (start 40 26.2937) (end 41.7854 26.2937) (width 0.3) (layer "F.Cu") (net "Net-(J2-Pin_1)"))
 (segment (start 41.7854 26.2937) (end 42.23 26.7383) (width 0.3) (layer "F.Cu") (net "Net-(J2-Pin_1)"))
 (segment (start 42.23 28.345) (end 42.23 26.7383) (width 0.3) (layer "F.Cu") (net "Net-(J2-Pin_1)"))
 (segment (start 40 26.2937) (end 36.7937 29.5) (width 0.3) (layer "F.Cu") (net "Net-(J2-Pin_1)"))
 (segment (start 31.625600 24.789900) (end 31.605700 24.770000) (width 0.25) (layer "F.Cu") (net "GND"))
 (segment (start 31.879100 28.975800) (end 31.679100 29.175800) (width 0.25) (layer "F.Cu") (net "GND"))
 (segment (start 29.250000 27.626700) (end 29.450000 27.826700) (width 0.5) (layer "F.Cu") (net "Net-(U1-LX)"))
 (segment (start 21.845000 24.570000) (end 21.845 21.5) (width 0.5) (layer "F.Cu") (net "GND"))
 (segment (start 21.845 21.5) (end 22.345 21.0) (width 0.5) (layer "F.Cu") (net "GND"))
 (segment (start 22.345 21.0) (end 39.5 21.0) (width 0.5) (layer "F.Cu") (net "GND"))
 (segment (start 39.5 21.0) (end 40.0 21.5) (width 0.5) (layer "F.Cu") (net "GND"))
 (segment (start 40.0 21.5) (end 40.000000 22.562500) (width 0.5) (layer "F.Cu") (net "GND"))
 (segment (start 22.045000 24.770000) (end 21.845000 24.570000) (width 0.25) (layer "F.Cu") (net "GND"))
 (segment (start 39.800000 22.762500) (end 40.000000 22.562500) (width 0.25) (layer "F.Cu") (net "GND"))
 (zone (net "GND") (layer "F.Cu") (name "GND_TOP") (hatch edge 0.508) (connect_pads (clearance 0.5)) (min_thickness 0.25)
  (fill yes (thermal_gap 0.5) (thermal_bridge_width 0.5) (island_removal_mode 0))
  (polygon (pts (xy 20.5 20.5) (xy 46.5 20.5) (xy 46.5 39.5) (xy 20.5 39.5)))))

